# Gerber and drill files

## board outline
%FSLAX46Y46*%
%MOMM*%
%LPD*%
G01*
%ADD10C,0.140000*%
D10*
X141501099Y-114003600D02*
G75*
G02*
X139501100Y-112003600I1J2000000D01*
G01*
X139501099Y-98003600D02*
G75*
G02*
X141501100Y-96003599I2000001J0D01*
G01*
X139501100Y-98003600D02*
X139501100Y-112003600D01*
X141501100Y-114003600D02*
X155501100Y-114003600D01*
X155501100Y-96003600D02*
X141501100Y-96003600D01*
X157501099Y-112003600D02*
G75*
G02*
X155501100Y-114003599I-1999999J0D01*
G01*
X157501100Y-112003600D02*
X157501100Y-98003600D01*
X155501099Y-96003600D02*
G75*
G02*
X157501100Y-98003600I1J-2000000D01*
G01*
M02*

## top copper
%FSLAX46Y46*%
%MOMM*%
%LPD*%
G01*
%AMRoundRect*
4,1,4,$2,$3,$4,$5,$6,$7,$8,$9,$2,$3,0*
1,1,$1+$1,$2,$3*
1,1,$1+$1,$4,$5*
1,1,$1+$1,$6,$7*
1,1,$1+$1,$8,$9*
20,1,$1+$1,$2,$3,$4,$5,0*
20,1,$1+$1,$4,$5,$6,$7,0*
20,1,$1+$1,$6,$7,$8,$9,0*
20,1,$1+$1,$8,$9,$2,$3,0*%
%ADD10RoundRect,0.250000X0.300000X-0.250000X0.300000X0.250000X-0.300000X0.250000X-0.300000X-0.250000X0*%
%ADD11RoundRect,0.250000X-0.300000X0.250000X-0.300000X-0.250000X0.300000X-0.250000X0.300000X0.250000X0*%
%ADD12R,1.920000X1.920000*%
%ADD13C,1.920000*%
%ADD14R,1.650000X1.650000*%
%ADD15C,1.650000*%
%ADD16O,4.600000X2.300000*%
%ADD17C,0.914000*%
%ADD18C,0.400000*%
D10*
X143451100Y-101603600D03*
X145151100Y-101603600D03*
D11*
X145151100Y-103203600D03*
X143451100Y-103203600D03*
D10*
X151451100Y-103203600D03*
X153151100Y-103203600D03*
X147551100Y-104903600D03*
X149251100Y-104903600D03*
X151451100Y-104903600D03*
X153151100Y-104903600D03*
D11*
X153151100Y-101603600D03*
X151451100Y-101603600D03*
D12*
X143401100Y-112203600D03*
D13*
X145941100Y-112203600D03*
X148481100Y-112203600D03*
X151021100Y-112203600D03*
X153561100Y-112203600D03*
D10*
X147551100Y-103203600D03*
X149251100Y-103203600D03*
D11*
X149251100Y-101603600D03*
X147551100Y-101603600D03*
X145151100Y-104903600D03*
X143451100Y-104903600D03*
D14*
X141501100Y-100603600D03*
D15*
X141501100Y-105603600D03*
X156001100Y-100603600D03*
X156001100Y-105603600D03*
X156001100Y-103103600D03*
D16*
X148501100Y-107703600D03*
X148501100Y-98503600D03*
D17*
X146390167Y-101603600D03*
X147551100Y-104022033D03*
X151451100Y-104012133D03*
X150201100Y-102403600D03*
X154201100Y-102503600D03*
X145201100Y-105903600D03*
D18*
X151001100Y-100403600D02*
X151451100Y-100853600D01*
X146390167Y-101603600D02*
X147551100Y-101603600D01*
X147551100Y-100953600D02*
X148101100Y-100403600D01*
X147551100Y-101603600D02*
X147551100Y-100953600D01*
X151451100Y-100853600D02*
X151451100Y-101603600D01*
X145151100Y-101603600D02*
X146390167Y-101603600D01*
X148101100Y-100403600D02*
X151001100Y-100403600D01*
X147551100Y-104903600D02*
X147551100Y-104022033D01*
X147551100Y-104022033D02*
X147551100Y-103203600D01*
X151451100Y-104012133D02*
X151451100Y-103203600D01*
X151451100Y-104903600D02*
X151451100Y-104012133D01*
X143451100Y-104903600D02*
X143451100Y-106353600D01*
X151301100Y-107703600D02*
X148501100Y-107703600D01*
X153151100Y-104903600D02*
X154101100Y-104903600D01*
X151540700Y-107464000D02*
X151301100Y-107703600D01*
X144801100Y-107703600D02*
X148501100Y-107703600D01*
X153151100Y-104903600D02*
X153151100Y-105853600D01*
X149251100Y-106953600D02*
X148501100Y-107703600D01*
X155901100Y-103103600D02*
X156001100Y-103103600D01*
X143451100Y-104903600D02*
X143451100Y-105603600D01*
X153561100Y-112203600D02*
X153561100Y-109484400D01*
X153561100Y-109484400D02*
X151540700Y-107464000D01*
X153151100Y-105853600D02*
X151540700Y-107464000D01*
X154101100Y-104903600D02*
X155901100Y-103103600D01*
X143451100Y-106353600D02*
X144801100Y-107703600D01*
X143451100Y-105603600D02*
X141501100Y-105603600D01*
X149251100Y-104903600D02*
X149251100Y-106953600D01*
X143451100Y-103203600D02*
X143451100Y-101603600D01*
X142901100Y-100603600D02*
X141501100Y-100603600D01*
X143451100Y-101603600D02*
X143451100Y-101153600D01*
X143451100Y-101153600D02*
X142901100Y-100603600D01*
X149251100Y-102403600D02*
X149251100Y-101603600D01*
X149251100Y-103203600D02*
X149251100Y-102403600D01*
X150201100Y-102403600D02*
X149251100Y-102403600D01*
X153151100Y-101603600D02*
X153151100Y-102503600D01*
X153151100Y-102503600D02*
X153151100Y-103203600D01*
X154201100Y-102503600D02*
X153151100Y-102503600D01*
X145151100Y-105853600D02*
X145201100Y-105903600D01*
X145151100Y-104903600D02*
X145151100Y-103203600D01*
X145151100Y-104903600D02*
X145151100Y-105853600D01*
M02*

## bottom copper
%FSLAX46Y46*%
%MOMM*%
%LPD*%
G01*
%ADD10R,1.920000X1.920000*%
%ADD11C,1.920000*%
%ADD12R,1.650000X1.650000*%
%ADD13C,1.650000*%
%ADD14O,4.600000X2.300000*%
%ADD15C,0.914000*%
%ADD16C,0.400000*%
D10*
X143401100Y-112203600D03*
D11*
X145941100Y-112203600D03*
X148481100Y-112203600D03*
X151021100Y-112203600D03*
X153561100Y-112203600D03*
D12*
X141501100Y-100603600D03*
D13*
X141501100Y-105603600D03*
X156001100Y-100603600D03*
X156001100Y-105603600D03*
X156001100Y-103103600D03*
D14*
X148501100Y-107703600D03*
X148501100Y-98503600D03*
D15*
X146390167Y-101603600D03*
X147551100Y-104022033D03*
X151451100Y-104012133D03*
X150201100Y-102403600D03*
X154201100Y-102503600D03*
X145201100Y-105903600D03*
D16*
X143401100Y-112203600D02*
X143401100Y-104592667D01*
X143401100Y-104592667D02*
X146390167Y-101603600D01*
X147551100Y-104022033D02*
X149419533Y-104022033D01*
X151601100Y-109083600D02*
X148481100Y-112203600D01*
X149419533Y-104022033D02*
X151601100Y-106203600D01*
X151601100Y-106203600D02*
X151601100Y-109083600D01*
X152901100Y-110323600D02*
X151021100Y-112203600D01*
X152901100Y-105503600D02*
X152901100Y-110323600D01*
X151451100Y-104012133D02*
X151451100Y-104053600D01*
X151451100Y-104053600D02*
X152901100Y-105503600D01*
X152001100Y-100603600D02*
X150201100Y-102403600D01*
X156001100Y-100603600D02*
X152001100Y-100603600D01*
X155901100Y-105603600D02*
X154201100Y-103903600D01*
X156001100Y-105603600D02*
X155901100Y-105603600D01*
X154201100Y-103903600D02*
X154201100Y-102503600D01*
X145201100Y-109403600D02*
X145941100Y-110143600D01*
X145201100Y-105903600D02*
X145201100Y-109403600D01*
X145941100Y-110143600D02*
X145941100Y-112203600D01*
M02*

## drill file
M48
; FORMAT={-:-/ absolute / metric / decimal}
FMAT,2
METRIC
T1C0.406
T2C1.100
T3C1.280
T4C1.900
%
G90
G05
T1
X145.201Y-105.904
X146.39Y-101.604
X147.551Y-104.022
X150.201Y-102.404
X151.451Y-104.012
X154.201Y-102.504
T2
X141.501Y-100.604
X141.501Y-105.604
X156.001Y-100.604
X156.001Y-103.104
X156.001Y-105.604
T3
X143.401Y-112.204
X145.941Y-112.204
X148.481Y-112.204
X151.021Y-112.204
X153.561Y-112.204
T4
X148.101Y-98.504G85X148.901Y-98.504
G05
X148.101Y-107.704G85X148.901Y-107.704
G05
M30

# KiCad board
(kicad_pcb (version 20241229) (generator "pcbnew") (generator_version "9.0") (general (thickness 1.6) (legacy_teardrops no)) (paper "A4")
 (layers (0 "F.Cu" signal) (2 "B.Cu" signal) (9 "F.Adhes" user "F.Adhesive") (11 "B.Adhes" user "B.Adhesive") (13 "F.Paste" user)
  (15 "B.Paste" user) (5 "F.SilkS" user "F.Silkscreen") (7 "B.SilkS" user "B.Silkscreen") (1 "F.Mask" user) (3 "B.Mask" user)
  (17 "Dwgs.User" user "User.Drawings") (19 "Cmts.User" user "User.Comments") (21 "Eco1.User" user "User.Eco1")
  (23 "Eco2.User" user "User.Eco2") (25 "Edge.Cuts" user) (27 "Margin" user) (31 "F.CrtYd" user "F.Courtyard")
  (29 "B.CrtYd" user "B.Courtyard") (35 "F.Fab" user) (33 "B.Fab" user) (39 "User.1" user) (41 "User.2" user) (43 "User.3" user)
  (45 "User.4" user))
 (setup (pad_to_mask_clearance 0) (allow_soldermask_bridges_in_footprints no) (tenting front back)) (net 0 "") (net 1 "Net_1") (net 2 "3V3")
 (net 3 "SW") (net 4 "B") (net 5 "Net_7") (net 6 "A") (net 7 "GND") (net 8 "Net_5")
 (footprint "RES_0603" (layer "F.Cu") (at 144.3011 101.6036)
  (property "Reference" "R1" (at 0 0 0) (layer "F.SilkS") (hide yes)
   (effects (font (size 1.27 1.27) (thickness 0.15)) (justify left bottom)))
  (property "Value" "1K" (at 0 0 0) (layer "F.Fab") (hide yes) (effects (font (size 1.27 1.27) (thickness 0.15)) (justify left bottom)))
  (pad "1" smd roundrect (at -0.85 0 90) (size 1 1.1) (layers "F.Cu" "F.Mask" "F.Paste") (roundrect_rratio 0.25) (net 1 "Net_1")
   (solder_mask_margin 0.0254) (solder_paste_margin -0.0254) (zone_connect 2) (thermal_bridge_angle 0))
  (pad "2" smd roundrect (at 0.85 0 90) (size 1 1.1) (layers "F.Cu" "F.Mask" "F.Paste") (roundrect_rratio 0.25) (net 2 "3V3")
   (solder_mask_margin 0.0254) (solder_paste_margin -0.0254) (zone_connect 2) (thermal_bridge_angle 0)))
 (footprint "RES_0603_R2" (layer "F.Cu") (at 144.3011 103.2036 180)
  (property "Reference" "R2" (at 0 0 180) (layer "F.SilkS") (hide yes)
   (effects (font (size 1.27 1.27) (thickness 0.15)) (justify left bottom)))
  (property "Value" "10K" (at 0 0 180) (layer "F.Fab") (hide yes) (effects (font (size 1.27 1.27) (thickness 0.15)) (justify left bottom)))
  (pad "1" smd roundrect (at -0.85 0 270) (size 1 1.1) (layers "F.Cu" "F.Mask" "F.Paste") (roundrect_rratio 0.25) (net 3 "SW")
   (solder_mask_margin 0.0254) (solder_paste_margin -0.0254) (zone_connect 2) (thermal_bridge_angle 0))
  (pad "2" smd roundrect (at 0.85 0 270) (size 1 1.1) (layers "F.Cu" "F.Mask" "F.Paste") (roundrect_rratio 0.25) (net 1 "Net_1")
   (solder_mask_margin 0.0254) (solder_paste_margin -0.0254) (zone_connect 2) (thermal_bridge_angle 0)))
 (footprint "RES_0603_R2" (layer "F.Cu") (at 152.3011 103.2036)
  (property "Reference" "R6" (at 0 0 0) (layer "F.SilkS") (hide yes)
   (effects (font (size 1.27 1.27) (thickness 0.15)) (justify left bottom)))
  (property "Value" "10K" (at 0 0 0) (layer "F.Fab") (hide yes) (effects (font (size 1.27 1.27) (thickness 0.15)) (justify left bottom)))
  (pad "1" smd roundrect (at -0.85 0 90) (size 1 1.1) (layers "F.Cu" "F.Mask" "F.Paste") (roundrect_rratio 0.25) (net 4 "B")
   (solder_mask_margin 0.0254) (solder_paste_margin -0.0254) (zone_connect 2) (thermal_bridge_angle 0))
  (pad "2" smd roundrect (at 0.85 0 90) (size 1 1.1) (layers "F.Cu" "F.Mask" "F.Paste") (roundrect_rratio 0.25) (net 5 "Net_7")
   (solder_mask_margin 0.0254) (solder_paste_margin -0.0254) (zone_connect 2) (thermal_bridge_angle 0)))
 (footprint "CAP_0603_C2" (layer "F.Cu") (at 148.4011 104.9036)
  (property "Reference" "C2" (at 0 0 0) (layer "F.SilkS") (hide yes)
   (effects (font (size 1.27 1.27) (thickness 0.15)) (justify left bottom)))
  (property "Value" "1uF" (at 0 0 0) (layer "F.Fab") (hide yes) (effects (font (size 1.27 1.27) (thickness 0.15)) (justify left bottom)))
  (pad "1" smd roundrect (at -0.85 0 90) (size 1 1.1) (layers "F.Cu" "F.Mask" "F.Paste") (roundrect_rratio 0.25) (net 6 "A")
   (solder_mask_margin 0.0254) (solder_paste_margin -0.0254) (zone_connect 2) (thermal_bridge_angle 0))
  (pad "2" smd roundrect (at 0.85 0 90) (size 1 1.1) (layers "F.Cu" "F.Mask" "F.Paste") (roundrect_rratio 0.25) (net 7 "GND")
   (solder_mask_margin 0.0254) (solder_paste_margin -0.0254) (zone_connect 2) (thermal_bridge_angle 0)))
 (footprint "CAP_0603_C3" (layer "F.Cu") (at 152.3011 104.9036)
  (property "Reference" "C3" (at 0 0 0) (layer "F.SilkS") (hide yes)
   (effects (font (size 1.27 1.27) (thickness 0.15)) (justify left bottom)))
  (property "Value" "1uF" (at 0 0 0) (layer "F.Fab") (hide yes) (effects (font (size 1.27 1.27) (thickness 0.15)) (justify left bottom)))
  (pad "1" smd roundrect (at -0.85 0 90) (size 1 1.1) (layers "F.Cu" "F.Mask" "F.Paste") (roundrect_rratio 0.25) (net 4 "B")
   (solder_mask_margin 0.0254) (solder_paste_margin -0.0254) (zone_connect 2) (thermal_bridge_angle 0))
  (pad "2" smd roundrect (at 0.85 0 90) (size 1 1.1) (layers "F.Cu" "F.Mask" "F.Paste") (roundrect_rratio 0.25) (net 7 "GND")
   (solder_mask_margin 0.0254) (solder_paste_margin -0.0254) (zone_connect 2) (thermal_bridge_angle 0)))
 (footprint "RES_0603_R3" (layer "F.Cu") (at 152.3011 101.6036 180)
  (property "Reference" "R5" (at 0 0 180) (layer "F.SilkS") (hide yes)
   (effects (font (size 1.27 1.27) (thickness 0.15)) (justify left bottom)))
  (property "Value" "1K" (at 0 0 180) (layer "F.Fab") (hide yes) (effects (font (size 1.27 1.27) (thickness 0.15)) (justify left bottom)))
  (pad "1" smd roundrect (at -0.85 0 270) (size 1 1.1) (layers "F.Cu" "F.Mask" "F.Paste") (roundrect_rratio 0.25) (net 5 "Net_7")
   (solder_mask_margin 0.0254) (solder_paste_margin -0.0254) (zone_connect 2) (thermal_bridge_angle 0))
  (pad "2" smd roundrect (at 0.85 0 270) (size 1 1.1) (layers "F.Cu" "F.Mask" "F.Paste") (roundrect_rratio 0.25) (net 2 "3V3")
   (solder_mask_margin 0.0254) (solder_paste_margin -0.0254) (zone_connect 2) (thermal_bridge_angle 0)))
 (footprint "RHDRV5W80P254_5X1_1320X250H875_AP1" (layer "F.Cu") (at 143.4011 112.2036)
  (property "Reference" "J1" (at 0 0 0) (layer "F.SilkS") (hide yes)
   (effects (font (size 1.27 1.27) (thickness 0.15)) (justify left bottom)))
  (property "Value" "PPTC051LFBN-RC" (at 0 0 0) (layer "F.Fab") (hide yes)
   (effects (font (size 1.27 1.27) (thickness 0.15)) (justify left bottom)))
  (pad "1" thru_hole rect (at 0 0 180) (size 1.92 1.92) (drill 1.28) (layers "*.Cu" "*.Mask") (remove_unused_layers no) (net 2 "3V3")
   (solder_mask_margin 0.0254) (zone_connect 2) (thermal_bridge_angle 0))
  (pad "2" thru_hole circle (at 2.54 0 180) (size 1.92 1.92) (drill 1.28) (layers "*.Cu" "*.Mask") (remove_unused_layers no) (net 3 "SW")
   (solder_mask_margin 0.0254) (zone_connect 2) (thermal_bridge_angle 0))
  (pad "3" thru_hole circle (at 5.08 0 180) (size 1.92 1.92) (drill 1.28) (layers "*.Cu" "*.Mask") (remove_unused_layers no) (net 6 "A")
   (solder_mask_margin 0.0254) (zone_connect 2) (thermal_bridge_angle 0))
  (pad "4" thru_hole circle (at 7.62 0 180) (size 1.92 1.92) (drill 1.28) (layers "*.Cu" "*.Mask") (remove_unused_layers no) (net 4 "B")
   (solder_mask_margin 0.0254) (zone_connect 2) (thermal_bridge_angle 0))
  (pad "5" thru_hole circle (at 10.16 0 180) (size 1.92 1.92) (drill 1.28) (layers "*.Cu" "*.Mask") (remove_unused_layers no) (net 7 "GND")
   (solder_mask_margin 0.0254) (zone_connect 2) (thermal_bridge_angle 0)))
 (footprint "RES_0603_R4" (layer "F.Cu") (at 148.4011 103.2036)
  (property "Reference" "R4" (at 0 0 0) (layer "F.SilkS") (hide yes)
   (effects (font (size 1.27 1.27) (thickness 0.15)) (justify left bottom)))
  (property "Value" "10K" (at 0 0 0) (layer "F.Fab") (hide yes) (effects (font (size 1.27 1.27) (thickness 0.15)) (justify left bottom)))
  (pad "1" smd roundrect (at -0.85 0 90) (size 1 1.1) (layers "F.Cu" "F.Mask" "F.Paste") (roundrect_rratio 0.25) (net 6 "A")
   (solder_mask_margin 0.0254) (solder_paste_margin -0.0254) (zone_connect 2) (thermal_bridge_angle 0))
  (pad "2" smd roundrect (at 0.85 0 90) (size 1 1.1) (layers "F.Cu" "F.Mask" "F.Paste") (roundrect_rratio 0.25) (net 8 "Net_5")
   (solder_mask_margin 0.0254) (solder_paste_margin -0.0254) (zone_connect 2) (thermal_bridge_angle 0)))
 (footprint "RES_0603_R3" (layer "F.Cu") (at 148.4011 101.6036 180)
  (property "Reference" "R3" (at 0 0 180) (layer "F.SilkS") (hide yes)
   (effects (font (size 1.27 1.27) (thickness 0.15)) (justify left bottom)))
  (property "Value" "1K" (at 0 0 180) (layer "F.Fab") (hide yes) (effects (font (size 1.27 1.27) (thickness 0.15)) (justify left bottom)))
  (pad "1" smd roundrect (at -0.85 0 270) (size 1 1.1) (layers "F.Cu" "F.Mask" "F.Paste") (roundrect_rratio 0.25) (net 8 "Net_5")
   (solder_mask_margin 0.0254) (solder_paste_margin -0.0254) (zone_connect 2) (thermal_bridge_angle 0))
  (pad "2" smd roundrect (at 0.85 0 270) (size 1 1.1) (layers "F.Cu" "F.Mask" "F.Paste") (roundrect_rratio 0.25) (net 2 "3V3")
   (solder_mask_margin 0.0254) (solder_paste_margin -0.0254) (zone_connect 2) (thermal_bridge_angle 0)))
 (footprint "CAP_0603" (layer "F.Cu") (at 144.3011 104.9036 180)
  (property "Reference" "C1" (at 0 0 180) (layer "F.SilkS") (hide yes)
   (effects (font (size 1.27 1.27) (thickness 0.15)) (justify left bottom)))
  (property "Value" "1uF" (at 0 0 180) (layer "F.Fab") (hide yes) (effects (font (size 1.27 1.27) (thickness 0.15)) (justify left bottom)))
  (pad "1" smd roundrect (at -0.85 0 270) (size 1 1.1) (layers "F.Cu" "F.Mask" "F.Paste") (roundrect_rratio 0.25) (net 3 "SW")
   (solder_mask_margin 0.0254) (solder_paste_margin -0.0254) (zone_connect 2) (thermal_bridge_angle 0))
  (pad "2" smd roundrect (at 0.85 0 270) (size 1 1.1) (layers "F.Cu" "F.Mask" "F.Paste") (roundrect_rratio 0.25) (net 7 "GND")
   (solder_mask_margin 0.0254) (solder_paste_margin -0.0254) (zone_connect 2) (thermal_bridge_angle 0)))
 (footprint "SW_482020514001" (layer "B.Cu") (at 148.5011 103.1036 -90)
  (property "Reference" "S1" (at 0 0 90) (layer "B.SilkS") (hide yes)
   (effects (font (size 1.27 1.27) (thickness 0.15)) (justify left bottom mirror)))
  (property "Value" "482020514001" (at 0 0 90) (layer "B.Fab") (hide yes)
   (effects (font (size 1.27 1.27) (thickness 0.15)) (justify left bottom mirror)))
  (pad "1" thru_hole rect (at -2.5 7 270) (size 1.65 1.65) (drill 1.1) (layers "*.Cu" "*.Mask") (remove_unused_layers no) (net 1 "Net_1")
   (solder_mask_margin 0.0254) (zone_connect 2) (thermal_bridge_angle 0))
  (pad "2" thru_hole circle (at 2.5 7 270) (size 1.65 1.65) (drill 1.1) (layers "*.Cu" "*.Mask") (remove_unused_layers no) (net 7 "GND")
   (solder_mask_margin 0.0254) (zone_connect 2) (thermal_bridge_angle 0))
  (pad "A" thru_hole circle (at -2.5 -7.5 270) (size 1.65 1.65) (drill 1.1) (layers "*.Cu" "*.Mask") (remove_unused_layers no)
   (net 8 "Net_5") (solder_mask_margin 0.0254) (zone_connect 2) (thermal_bridge_angle 0))
  (pad "B" thru_hole circle (at 2.5 -7.5 270) (size 1.65 1.65) (drill 1.1) (layers "*.Cu" "*.Mask") (remove_unused_layers no)
   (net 5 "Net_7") (solder_mask_margin 0.0254) (zone_connect 2) (thermal_bridge_angle 0))
  (pad "C" thru_hole circle (at 0 -7.5 270) (size 1.65 1.65) (drill 1.1) (layers "*.Cu" "*.Mask") (remove_unused_layers no) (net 7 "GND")
   (solder_mask_margin 0.0254) (zone_connect 2) (thermal_bridge_angle 0))
  (pad "S1" thru_hole oval (at 4.6 0) (size 4.6 2.3) (drill oval 2.7 1.9) (layers "*.Cu" "*.Mask") (remove_unused_layers no) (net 7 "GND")
   (solder_mask_margin 0.0254) (zone_connect 2) (thermal_bridge_angle 0))
  (pad "S2" thru_hole oval (at -4.6 0) (size 4.6 2.3) (drill oval 2.7 1.9) (layers "*.Cu" "*.Mask") (remove_unused_layers no) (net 7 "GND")
   (solder_mask_margin 0.0254) (zone_connect 2) (thermal_bridge_angle 0)))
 (gr_arc (start 141.501099 114.0036) (mid 140.0869 113.4178) (end 139.5011 112.0036) (stroke (width 0.14) (type solid)) (layer "Edge.Cuts"))
 (gr_arc (start 139.501099 98.0036) (mid 140.0869 96.5894) (end 141.5011 96.0036) (stroke (width 0.14) (type solid)) (layer "Edge.Cuts"))
 (gr_line (start 139.5011 98.0036) (end 139.5011 112.0036) (stroke (width 0.14) (type solid)) (layer "Edge.Cuts"))
 (gr_line (start 141.5011 114.0036) (end 155.5011 114.0036) (stroke (width 0.14) (type solid)) (layer "Edge.Cuts"))
 (gr_line (start 155.5011 96.0036) (end 141.5011 96.0036) (stroke (width 0.14) (type solid)) (layer "Edge.Cuts"))
 (gr_arc (start 157.501099 112.0036) (mid 156.915299 113.4178) (end 155.5011 114.0036) (stroke (width 0.14) (type solid))
  (layer "Edge.Cuts"))
 (gr_line (start 157.5011 112.0036) (end 157.5011 98.0036) (stroke (width 0.14) (type solid)) (layer "Edge.Cuts"))
 (gr_arc (start 155.501099 96.0036) (mid 156.915299 96.5894) (end 157.5011 98.0036) (stroke (width 0.14) (type solid)) (layer "Edge.Cuts"))
 (segment (start 151.0011 100.4036) (end 151.4511 100.8536) (width 0.4) (layer "F.Cu") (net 2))
 (segment (start 146.390167 101.6036) (end 147.5511 101.6036) (width 0.4) (layer "F.Cu") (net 2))
 (segment (start 147.5511 100.9536) (end 148.1011 100.4036) (width 0.4) (layer "F.Cu") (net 2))
 (segment (start 147.5511 101.6036) (end 147.5511 100.9536) (width 0.4) (layer "F.Cu") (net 2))
 (segment (start 151.4511 100.8536) (end 151.4511 101.6036) (width 0.4) (layer "F.Cu") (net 2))
 (segment (start 145.1511 101.6036) (end 146.390167 101.6036) (width 0.4) (layer "F.Cu") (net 2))
 (segment (start 148.1011 100.4036) (end 151.0011 100.4036) (width 0.4) (layer "F.Cu") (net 2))
 (via (at 146.390167 101.6036) (size 0.914) (drill 0.406) (layers "F.Cu" "B.Cu") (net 2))
 (segment (start 143.4011 112.2036) (end 143.4011 104.592667) (width 0.4) (layer "B.Cu") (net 2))
 (segment (start 143.4011 104.592667) (end 146.390167 101.6036) (width 0.4) (layer "B.Cu") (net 2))
 (segment (start 147.5511 104.9036) (end 147.5511 104.022033) (width 0.4) (layer "F.Cu") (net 6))
 (segment (start 147.5511 104.022033) (end 147.5511 103.2036) (width 0.4) (layer "F.Cu") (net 6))
 (via (at 147.5511 104.022033) (size 0.914) (drill 0.406) (layers "F.Cu" "B.Cu") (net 6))
 (segment (start 147.5511 104.022033) (end 149.419533 104.022033) (width 0.4) (layer "B.Cu") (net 6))
 (segment (start 151.6011 109.0836) (end 148.4811 112.2036) (width 0.4) (layer "B.Cu") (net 6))
 (segment (start 149.419533 104.022033) (end 151.6011 106.2036) (width 0.4) (layer "B.Cu") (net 6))
 (segment (start 151.6011 106.2036) (end 151.6011 109.0836) (width 0.4) (layer "B.Cu") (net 6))
 (segment (start 151.4511 104.012133) (end 151.4511 103.2036) (width 0.4) (layer "F.Cu") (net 4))
 (segment (start 151.4511 104.9036) (end 151.4511 104.012133) (width 0.4) (layer "F.Cu") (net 4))
 (via (at 151.4511 104.012133) (size 0.914) (drill 0.406) (layers "F.Cu" "B.Cu") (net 4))
 (segment (start 152.9011 110.3236) (end 151.0211 112.2036) (width 0.4) (layer "B.Cu") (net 4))
 (segment (start 152.9011 105.5036) (end 152.9011 110.3236) (width 0.4) (layer "B.Cu") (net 4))
 (segment (start 151.4511 104.012133) (end 151.4511 104.0536) (width 0.4) (layer "B.Cu") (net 4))
 (segment (start 151.4511 104.0536) (end 152.9011 105.5036) (width 0.4) (layer "B.Cu") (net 4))
 (segment (start 143.4511 104.9036) (end 143.4511 106.3536) (width 0.4) (layer "F.Cu") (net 7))
 (segment (start 151.3011 107.7036) (end 148.5011 107.7036) (width 0.4) (layer "F.Cu") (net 7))
 (segment (start 153.1511 104.9036) (end 154.1011 104.9036) (width 0.4) (layer "F.Cu") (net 7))
 (segment (start 151.5407 107.464) (end 151.3011 107.7036) (width 0.4) (layer "F.Cu") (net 7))
 (segment (start 144.8011 107.7036) (end 148.5011 107.7036) (width 0.4) (layer "F.Cu") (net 7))
 (segment (start 153.1511 104.9036) (end 153.1511 105.8536) (width 0.4) (layer "F.Cu") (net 7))
 (segment (start 149.2511 106.9536) (end 148.5011 107.7036) (width 0.4) (layer "F.Cu") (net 7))
 (segment (start 155.9011 103.1036) (end 156.0011 103.1036) (width 0.4) (layer "F.Cu") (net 7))
 (segment (start 143.4511 104.9036) (end 143.4511 105.6036) (width 0.4) (layer "F.Cu") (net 7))
 (segment (start 153.5611 112.2036) (end 153.5611 109.4844) (width 0.4) (layer "F.Cu") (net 7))
 (segment (start 153.5611 109.4844) (end 151.5407 107.464) (width 0.4) (layer "F.Cu") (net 7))
 (segment (start 153.1511 105.8536) (end 151.5407 107.464) (width 0.4) (layer "F.Cu") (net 7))
 (segment (start 154.1011 104.9036) (end 155.9011 103.1036) (width 0.4) (layer "F.Cu") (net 7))
 (segment (start 143.4511 106.3536) (end 144.8011 107.7036) (width 0.4) (layer "F.Cu") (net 7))
 (segment (start 143.4511 105.6036) (end 141.5011 105.6036) (width 0.4) (layer "F.Cu") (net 7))
 (segment (start 149.2511 104.9036) (end 149.2511 106.9536) (width 0.4) (layer "F.Cu") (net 7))
 (segment (start 143.4511 103.2036) (end 143.4511 101.6036) (width 0.4) (layer "F.Cu") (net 1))
 (segment (start 142.9011 100.6036) (end 141.5011 100.6036) (width 0.4) (layer "F.Cu") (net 1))
 (segment (start 143.4511 101.6036) (end 143.4511 101.1536) (width 0.4) (layer "F.Cu") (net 1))
 (segment (start 143.4511 101.1536) (end 142.9011 100.6036) (width 0.4) (layer "F.Cu") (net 1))
 (segment (start 149.2511 102.4036) (end 149.2511 101.6036) (width 0.4) (layer "F.Cu") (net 8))
 (segment (start 149.2511 103.2036) (end 149.2511 102.4036) (width 0.4) (layer "F.Cu") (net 8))
 (segment (start 150.2011 102.4036) (end 149.2511 102.4036) (width 0.4) (layer "F.Cu") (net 8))
 (via (at 150.2011 102.4036) (size 0.914) (drill 0.406) (layers "F.Cu" "B.Cu") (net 8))
 (segment (start 152.0011 100.6036) (end 150.2011 102.4036) (width 0.4) (layer "B.Cu") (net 8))
 (segment (start 156.0011 100.6036) (end 152.0011 100.6036) (width 0.4) (layer "B.Cu") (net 8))
 (segment (start 153.1511 101.6036) (end 153.1511 102.5036) (width 0.4) (layer "F.Cu") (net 5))
 (segment (start 153.1511 102.5036) (end 153.1511 103.2036) (width 0.4) (layer "F.Cu") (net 5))
 (segment (start 154.2011 102.5036) (end 153.1511 102.5036) (width 0.4) (layer "F.Cu") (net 5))
 (via (at 154.2011 102.5036) (size 0.914) (drill 0.406) (layers "F.Cu" "B.Cu") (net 5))
 (segment (start 155.9011 105.6036) (end 154.2011 103.9036) (width 0.4) (layer "B.Cu") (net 5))
 (segment (start 156.0011 105.6036) (end 155.9011 105.6036) (width 0.4) (layer "B.Cu") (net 5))
 (segment (start 154.2011 103.9036) (end 154.2011 102.5036) (width 0.4) (layer "B.Cu") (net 5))
 (segment (start 145.1511 105.8536) (end 145.2011 105.9036) (width 0.4) (layer "F.Cu") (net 3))
 (segment (start 145.1511 104.9036) (end 145.1511 103.2036) (width 0.4) (layer "F.Cu") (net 3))
 (segment (start 145.1511 104.9036) (end 145.1511 105.8536) (width 0.4) (layer "F.Cu") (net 3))
 (via (at 145.2011 105.9036) (size 0.914) (drill 0.406) (layers "F.Cu" "B.Cu") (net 3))
 (segment (start 145.2011 109.4036) (end 145.9411 110.1436) (width 0.4) (layer "B.Cu") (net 3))
 (segment (start 145.2011 105.9036) (end 145.2011 109.4036) (width 0.4) (layer "B.Cu") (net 3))
 (segment (start 145.9411 110.1436) (end 145.9411 112.2036) (width 0.4) (layer "B.Cu") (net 3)))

